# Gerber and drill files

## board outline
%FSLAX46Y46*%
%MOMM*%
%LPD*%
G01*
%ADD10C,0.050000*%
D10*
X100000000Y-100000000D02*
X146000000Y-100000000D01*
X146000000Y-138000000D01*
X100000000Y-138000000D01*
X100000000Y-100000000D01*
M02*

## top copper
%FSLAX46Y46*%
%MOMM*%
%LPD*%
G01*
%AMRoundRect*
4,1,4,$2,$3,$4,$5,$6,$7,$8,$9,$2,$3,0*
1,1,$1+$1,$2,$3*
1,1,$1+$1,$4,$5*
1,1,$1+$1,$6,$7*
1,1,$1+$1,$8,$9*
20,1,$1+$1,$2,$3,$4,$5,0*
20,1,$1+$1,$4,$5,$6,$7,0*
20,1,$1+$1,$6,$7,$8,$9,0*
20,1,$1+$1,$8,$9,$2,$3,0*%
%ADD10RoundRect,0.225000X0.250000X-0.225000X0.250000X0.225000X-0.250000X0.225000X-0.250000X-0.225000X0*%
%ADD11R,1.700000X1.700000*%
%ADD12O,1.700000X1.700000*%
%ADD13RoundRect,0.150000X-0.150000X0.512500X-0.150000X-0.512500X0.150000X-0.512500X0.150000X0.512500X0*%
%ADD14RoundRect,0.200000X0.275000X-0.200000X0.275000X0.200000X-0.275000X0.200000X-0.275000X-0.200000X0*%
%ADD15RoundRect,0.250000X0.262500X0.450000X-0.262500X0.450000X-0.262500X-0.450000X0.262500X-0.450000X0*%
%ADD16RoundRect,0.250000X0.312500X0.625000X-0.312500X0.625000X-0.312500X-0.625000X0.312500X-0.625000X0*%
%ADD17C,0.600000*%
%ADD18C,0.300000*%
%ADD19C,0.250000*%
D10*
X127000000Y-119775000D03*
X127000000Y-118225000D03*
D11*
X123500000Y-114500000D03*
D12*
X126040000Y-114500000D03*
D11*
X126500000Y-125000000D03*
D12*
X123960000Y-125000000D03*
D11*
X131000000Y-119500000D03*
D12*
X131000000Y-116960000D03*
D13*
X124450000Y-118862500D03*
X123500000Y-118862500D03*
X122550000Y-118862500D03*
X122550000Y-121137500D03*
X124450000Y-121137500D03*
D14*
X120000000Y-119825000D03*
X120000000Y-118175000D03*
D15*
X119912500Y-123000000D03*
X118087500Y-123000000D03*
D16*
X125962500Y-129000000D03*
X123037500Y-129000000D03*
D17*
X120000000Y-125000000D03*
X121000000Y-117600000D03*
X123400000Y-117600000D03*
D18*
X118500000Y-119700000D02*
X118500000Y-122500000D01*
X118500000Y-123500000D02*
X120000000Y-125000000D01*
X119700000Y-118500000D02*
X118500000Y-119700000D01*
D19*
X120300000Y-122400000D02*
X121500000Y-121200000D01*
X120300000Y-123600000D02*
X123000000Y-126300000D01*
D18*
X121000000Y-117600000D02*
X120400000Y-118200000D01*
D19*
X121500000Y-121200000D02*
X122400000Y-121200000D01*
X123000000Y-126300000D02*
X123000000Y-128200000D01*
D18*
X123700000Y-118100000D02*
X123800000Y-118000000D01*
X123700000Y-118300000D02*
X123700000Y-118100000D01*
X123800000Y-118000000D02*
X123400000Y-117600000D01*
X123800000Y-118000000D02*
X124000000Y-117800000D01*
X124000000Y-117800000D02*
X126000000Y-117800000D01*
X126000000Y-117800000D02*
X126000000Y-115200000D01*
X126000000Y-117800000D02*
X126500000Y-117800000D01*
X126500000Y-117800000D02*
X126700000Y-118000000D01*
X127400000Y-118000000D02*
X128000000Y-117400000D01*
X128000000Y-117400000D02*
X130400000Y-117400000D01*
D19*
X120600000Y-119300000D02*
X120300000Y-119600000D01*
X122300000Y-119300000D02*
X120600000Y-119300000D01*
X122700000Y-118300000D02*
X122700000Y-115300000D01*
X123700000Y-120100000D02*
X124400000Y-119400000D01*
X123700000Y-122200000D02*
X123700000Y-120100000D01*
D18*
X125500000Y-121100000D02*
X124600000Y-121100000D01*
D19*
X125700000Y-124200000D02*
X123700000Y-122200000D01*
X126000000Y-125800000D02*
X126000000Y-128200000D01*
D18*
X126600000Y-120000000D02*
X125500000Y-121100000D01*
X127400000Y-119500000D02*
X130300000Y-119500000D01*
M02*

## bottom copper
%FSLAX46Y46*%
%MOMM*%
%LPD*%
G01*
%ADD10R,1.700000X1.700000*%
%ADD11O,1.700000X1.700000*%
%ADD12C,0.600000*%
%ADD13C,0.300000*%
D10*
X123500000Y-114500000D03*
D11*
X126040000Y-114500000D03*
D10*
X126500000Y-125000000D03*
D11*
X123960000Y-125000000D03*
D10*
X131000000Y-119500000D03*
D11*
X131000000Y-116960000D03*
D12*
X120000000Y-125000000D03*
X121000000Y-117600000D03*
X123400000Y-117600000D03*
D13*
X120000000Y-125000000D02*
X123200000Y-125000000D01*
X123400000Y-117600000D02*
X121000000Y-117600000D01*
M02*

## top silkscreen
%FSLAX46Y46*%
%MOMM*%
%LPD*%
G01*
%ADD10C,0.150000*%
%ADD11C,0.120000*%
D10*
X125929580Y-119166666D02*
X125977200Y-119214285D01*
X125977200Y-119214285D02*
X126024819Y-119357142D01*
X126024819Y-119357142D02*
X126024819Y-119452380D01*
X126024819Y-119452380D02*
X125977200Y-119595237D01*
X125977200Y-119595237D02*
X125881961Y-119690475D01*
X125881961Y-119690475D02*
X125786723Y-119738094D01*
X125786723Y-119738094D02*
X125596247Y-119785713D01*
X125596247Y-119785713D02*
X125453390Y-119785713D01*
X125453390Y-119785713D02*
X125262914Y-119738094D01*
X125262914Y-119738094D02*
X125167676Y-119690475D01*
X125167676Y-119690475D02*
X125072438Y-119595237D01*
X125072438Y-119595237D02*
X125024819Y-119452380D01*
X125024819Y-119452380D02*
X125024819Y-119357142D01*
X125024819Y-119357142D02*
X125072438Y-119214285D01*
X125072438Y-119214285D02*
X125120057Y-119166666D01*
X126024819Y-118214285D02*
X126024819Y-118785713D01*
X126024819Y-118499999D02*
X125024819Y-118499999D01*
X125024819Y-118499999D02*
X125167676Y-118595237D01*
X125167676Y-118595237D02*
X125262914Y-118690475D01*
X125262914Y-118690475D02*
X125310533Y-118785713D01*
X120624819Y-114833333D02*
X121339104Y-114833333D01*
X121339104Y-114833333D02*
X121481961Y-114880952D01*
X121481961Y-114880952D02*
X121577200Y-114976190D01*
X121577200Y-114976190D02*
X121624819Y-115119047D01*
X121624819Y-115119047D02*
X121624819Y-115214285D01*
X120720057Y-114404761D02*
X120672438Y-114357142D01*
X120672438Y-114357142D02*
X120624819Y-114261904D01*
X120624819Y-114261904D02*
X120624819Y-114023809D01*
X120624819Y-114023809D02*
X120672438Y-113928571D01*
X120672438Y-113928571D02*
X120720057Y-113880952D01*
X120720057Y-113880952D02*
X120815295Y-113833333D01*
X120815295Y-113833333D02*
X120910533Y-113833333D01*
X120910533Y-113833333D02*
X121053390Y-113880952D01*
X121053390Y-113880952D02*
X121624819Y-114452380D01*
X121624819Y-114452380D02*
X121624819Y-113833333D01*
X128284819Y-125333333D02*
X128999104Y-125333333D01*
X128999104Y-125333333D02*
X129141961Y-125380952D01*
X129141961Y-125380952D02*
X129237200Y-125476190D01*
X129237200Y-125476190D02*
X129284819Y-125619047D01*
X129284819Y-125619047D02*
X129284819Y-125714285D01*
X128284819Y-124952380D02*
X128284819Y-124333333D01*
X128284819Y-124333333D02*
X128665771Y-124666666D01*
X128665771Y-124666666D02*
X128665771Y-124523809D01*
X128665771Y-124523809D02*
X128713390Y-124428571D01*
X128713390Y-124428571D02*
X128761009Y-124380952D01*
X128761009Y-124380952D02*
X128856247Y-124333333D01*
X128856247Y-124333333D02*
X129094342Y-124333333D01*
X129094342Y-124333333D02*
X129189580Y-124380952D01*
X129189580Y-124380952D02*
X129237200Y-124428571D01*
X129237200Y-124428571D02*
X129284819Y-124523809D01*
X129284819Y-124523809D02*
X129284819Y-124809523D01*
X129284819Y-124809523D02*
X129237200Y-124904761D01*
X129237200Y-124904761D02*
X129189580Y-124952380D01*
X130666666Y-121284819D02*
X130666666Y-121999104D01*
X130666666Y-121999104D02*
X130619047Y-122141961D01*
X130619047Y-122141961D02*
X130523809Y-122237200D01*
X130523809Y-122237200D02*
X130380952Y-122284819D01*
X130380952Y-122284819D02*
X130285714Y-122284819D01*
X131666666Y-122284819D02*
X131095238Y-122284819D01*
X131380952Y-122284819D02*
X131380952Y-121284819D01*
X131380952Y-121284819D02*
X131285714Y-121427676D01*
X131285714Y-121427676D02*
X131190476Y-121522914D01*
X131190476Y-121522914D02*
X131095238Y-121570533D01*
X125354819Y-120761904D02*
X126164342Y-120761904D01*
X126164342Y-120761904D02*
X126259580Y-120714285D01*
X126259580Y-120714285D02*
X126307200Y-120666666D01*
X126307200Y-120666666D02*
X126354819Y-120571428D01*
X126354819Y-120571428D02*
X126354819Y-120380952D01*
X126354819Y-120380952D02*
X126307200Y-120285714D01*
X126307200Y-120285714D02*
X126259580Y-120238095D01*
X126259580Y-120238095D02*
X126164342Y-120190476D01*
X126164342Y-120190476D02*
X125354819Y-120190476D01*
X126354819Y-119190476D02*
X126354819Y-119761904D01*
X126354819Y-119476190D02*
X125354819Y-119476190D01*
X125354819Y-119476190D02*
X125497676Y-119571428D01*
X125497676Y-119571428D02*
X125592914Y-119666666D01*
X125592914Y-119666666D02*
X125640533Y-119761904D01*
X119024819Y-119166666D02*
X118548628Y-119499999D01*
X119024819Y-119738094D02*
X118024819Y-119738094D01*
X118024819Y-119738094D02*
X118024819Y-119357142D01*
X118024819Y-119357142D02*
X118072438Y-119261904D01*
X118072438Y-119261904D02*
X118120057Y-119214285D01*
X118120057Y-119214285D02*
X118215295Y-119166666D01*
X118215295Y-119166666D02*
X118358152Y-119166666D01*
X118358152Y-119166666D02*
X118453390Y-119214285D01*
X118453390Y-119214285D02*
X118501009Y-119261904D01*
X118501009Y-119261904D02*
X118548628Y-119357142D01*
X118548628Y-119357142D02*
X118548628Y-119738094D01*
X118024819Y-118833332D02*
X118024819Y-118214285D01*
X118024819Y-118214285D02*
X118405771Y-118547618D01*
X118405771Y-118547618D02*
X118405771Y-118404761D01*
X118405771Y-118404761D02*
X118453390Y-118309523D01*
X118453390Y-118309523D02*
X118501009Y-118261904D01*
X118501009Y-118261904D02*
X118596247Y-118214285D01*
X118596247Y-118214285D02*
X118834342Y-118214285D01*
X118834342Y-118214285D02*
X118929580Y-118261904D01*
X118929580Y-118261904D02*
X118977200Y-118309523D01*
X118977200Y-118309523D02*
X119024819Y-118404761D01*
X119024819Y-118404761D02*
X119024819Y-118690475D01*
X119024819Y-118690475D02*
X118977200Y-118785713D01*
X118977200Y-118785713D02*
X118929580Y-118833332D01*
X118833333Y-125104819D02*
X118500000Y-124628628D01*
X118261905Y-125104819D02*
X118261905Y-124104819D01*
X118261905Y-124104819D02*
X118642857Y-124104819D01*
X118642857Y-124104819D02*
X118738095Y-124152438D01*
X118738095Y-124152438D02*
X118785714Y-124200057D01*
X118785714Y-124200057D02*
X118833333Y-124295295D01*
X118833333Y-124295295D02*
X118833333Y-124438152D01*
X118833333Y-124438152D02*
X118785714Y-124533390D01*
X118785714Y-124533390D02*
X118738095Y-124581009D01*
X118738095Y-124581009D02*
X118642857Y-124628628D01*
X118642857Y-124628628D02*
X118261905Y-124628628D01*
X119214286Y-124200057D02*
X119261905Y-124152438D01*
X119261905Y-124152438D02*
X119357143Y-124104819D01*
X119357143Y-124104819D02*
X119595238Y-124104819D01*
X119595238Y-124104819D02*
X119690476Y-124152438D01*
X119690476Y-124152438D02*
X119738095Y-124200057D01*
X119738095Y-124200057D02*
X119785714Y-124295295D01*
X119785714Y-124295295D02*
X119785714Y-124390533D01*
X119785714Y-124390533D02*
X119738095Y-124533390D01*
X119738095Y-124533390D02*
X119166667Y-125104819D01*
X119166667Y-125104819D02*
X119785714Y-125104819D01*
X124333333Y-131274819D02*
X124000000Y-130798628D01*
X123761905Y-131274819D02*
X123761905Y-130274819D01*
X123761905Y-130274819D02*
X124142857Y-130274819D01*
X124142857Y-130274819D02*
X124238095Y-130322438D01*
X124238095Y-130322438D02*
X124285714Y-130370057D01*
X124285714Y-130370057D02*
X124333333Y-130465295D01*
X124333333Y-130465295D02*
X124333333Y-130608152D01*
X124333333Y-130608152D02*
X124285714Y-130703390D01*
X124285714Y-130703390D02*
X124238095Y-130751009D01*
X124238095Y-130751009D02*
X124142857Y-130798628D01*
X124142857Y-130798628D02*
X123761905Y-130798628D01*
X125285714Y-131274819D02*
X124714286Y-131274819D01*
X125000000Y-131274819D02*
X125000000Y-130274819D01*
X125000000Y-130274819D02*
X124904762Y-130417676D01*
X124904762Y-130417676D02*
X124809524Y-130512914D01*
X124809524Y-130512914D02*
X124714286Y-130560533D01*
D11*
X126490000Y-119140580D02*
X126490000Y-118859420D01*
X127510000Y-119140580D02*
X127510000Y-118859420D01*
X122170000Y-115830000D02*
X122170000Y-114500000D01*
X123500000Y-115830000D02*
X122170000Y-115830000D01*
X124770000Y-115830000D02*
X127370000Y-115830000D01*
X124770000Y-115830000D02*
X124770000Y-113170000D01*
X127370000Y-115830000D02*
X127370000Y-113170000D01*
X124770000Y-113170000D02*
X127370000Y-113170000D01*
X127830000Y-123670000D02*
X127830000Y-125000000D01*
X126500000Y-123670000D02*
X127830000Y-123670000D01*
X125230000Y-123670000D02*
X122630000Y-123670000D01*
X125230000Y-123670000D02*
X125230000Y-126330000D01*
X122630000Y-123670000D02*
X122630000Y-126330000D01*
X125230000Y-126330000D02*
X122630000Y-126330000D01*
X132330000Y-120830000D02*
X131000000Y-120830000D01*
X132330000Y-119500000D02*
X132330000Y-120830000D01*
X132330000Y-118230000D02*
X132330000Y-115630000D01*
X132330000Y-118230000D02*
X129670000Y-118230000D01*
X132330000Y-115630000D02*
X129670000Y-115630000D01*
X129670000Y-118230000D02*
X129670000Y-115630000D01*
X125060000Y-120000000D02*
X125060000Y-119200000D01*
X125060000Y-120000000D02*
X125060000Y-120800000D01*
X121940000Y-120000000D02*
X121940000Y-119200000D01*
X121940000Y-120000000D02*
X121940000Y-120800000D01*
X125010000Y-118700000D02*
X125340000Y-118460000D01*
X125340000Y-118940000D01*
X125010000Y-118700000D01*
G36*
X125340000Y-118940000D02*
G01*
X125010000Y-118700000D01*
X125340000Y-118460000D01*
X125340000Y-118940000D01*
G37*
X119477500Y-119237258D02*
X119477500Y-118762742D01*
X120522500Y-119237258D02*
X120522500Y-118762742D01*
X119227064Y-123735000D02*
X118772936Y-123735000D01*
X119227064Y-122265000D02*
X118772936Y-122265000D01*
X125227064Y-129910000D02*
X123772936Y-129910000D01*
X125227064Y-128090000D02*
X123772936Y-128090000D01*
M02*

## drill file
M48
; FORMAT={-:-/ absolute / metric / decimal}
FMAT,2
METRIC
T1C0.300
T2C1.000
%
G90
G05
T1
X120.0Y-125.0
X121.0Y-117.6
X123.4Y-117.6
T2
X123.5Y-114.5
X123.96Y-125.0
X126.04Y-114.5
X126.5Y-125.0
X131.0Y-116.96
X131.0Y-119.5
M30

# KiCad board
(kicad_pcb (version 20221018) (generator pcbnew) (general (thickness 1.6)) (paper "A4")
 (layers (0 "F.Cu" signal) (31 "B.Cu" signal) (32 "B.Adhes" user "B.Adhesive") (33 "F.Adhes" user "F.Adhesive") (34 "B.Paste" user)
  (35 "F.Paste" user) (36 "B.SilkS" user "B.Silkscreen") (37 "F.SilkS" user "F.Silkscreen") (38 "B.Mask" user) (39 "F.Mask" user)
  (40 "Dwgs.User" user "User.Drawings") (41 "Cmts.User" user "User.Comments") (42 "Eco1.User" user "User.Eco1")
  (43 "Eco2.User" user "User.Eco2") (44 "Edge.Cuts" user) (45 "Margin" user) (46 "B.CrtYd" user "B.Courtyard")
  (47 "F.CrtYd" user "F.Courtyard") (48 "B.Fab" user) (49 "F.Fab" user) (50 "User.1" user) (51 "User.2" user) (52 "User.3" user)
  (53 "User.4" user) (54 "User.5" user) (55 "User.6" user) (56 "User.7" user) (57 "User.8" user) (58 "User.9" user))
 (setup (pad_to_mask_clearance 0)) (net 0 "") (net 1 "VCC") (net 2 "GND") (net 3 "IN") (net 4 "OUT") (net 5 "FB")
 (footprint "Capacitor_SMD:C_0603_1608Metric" (layer "F.Cu") (at 127 119 90)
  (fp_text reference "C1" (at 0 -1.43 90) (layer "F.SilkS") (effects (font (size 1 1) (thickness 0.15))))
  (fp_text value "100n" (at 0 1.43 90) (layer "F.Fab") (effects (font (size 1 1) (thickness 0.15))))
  (fp_line (start -0.14058 -0.51) (end 0.14058 -0.51) (stroke (width 0.12) (type solid)) (layer "F.SilkS"))
  (fp_line (start -0.14058 0.51) (end 0.14058 0.51) (stroke (width 0.12) (type solid)) (layer "F.SilkS"))
  (pad "1" smd roundrect (at -0.775 0 90) (size 0.9 0.95) (layers "F.Cu" "F.Paste" "F.Mask") (roundrect_rratio 0.25) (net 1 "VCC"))
  (pad "2" smd roundrect (at 0.775 0 90) (size 0.9 0.95) (layers "F.Cu" "F.Paste" "F.Mask") (roundrect_rratio 0.25) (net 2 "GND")))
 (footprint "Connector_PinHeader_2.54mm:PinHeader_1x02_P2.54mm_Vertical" (layer "F.Cu") (at 123.5 114.5 90)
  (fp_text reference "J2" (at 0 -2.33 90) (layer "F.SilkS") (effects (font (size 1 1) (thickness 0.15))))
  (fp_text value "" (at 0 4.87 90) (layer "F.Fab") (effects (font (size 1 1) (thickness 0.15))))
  (fp_line (start -1.33 -1.33) (end 0 -1.33) (stroke (width 0.12) (type solid)) (layer "F.SilkS"))
  (fp_line (start -1.33 0) (end -1.33 -1.33) (stroke (width 0.12) (type solid)) (layer "F.SilkS"))
  (fp_line (start -1.33 1.27) (end -1.33 3.87) (stroke (width 0.12) (type solid)) (layer "F.SilkS"))
  (fp_line (start -1.33 1.27) (end 1.33 1.27) (stroke (width 0.12) (type solid)) (layer "F.SilkS"))
  (fp_line (start -1.33 3.87) (end 1.33 3.87) (stroke (width 0.12) (type solid)) (layer "F.SilkS"))
  (fp_line (start 1.33 1.27) (end 1.33 3.87) (stroke (width 0.12) (type solid)) (layer "F.SilkS"))
  (pad "1" thru_hole rect (at 0 0 90) (size 1.7 1.7) (drill 1) (layers "*.Cu" "*.Mask") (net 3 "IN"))
  (pad "2" thru_hole oval (at 0 2.54 90) (size 1.7 1.7) (drill 1) (layers "*.Cu" "*.Mask") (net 2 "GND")))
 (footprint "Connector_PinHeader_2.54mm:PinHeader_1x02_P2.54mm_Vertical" (layer "F.Cu") (at 126.5 125 -90)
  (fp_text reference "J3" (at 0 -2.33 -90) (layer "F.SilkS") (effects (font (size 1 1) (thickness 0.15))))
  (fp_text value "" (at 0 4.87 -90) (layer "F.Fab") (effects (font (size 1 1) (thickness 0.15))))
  (fp_line (start -1.33 -1.33) (end 0 -1.33) (stroke (width 0.12) (type solid)) (layer "F.SilkS"))
  (fp_line (start -1.33 0) (end -1.33 -1.33) (stroke (width 0.12) (type solid)) (layer "F.SilkS"))
  (fp_line (start -1.33 1.27) (end -1.33 3.87) (stroke (width 0.12) (type solid)) (layer "F.SilkS"))
  (fp_line (start -1.33 1.27) (end 1.33 1.27) (stroke (width 0.12) (type solid)) (layer "F.SilkS"))
  (fp_line (start -1.33 3.87) (end 1.33 3.87) (stroke (width 0.12) (type solid)) (layer "F.SilkS"))
  (fp_line (start 1.33 1.27) (end 1.33 3.87) (stroke (width 0.12) (type solid)) (layer "F.SilkS"))
  (pad "1" thru_hole rect (at 0 0 270) (size 1.7 1.7) (drill 1) (layers "*.Cu" "*.Mask") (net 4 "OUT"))
  (pad "2" thru_hole oval (at 0 2.54 270) (size 1.7 1.7) (drill 1) (layers "*.Cu" "*.Mask") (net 2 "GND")))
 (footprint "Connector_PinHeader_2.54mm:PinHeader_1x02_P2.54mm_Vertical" (layer "F.Cu") (at 131 119.5 180)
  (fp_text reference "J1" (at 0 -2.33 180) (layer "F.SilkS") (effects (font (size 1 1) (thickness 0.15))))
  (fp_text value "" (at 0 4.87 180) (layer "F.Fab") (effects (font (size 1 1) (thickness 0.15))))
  (fp_line (start -1.33 -1.33) (end 0 -1.33) (stroke (width 0.12) (type solid)) (layer "F.SilkS"))
  (fp_line (start -1.33 0) (end -1.33 -1.33) (stroke (width 0.12) (type solid)) (layer "F.SilkS"))
  (fp_line (start -1.33 1.27) (end -1.33 3.87) (stroke (width 0.12) (type solid)) (layer "F.SilkS"))
  (fp_line (start -1.33 1.27) (end 1.33 1.27) (stroke (width 0.12) (type solid)) (layer "F.SilkS"))
  (fp_line (start -1.33 3.87) (end 1.33 3.87) (stroke (width 0.12) (type solid)) (layer "F.SilkS"))
  (fp_line (start 1.33 1.27) (end 1.33 3.87) (stroke (width 0.12) (type solid)) (layer "F.SilkS"))
  (pad "1" thru_hole rect (at 0 0 180) (size 1.7 1.7) (drill 1) (layers "*.Cu" "*.Mask") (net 1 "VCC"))
  (pad "2" thru_hole oval (at 0 2.54 180) (size 1.7 1.7) (drill 1) (layers "*.Cu" "*.Mask") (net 2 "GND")))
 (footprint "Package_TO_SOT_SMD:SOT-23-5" (layer "F.Cu") (at 123.5 120 -90)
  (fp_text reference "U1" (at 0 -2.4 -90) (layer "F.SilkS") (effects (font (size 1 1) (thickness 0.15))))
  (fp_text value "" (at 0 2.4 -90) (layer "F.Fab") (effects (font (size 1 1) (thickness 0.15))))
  (fp_line (start 0 -1.56) (end -0.8 -1.56) (stroke (width 0.12) (type solid)) (layer "F.SilkS"))
  (fp_line (start 0 -1.56) (end 0.8 -1.56) (stroke (width 0.12) (type solid)) (layer "F.SilkS"))
  (fp_line (start 0 1.56) (end -0.8 1.56) (stroke (width 0.12) (type solid)) (layer "F.SilkS"))
  (fp_line (start 0 1.56) (end 0.8 1.56) (stroke (width 0.12) (type solid)) (layer "F.SilkS"))
  (fp_poly
   (pts (xy -1.3 -1.51) (xy -1.54 -1.84) (xy -1.06 -1.84) (xy -1.3 -1.51)) (stroke (width 0.12) (type solid)) (fill solid) (layer "F.SilkS"))
  (pad "1" smd roundrect (at -1.1375 -0.95 270) (size 1.325 0.6) (layers "F.Cu" "F.Paste" "F.Mask") (roundrect_rratio 0.25) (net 4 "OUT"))
  (pad "2" smd roundrect (at -1.1375 0 270) (size 1.325 0.6) (layers "F.Cu" "F.Paste" "F.Mask") (roundrect_rratio 0.25) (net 2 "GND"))
  (pad "3" smd roundrect (at -1.1375 0.95 270) (size 1.325 0.6) (layers "F.Cu" "F.Paste" "F.Mask") (roundrect_rratio 0.25) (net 3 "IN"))
  (pad "4" smd roundrect (at 1.1375 0.95 270) (size 1.325 0.6) (layers "F.Cu" "F.Paste" "F.Mask") (roundrect_rratio 0.25) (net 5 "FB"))
  (pad "5" smd roundrect (at 1.1375 -0.95 270) (size 1.325 0.6) (layers "F.Cu" "F.Paste" "F.Mask") (roundrect_rratio 0.25) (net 1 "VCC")))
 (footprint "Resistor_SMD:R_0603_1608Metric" (layer "F.Cu") (at 120 119 90)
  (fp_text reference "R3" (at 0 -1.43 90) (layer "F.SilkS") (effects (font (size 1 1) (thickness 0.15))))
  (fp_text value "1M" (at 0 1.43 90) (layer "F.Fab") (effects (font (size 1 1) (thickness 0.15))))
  (fp_line (start -0.237258 -0.5225) (end 0.237258 -0.5225) (stroke (width 0.12) (type solid)) (layer "F.SilkS"))
  (fp_line (start -0.237258 0.5225) (end 0.237258 0.5225) (stroke (width 0.12) (type solid)) (layer "F.SilkS"))
  (pad "1" smd roundrect (at -0.825 0 90) (size 0.8 0.95) (layers "F.Cu" "F.Paste" "F.Mask") (roundrect_rratio 0.25) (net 3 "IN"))
  (pad "2" smd roundrect (at 0.825 0 90) (size 0.8 0.95) (layers "F.Cu" "F.Paste" "F.Mask") (roundrect_rratio 0.25) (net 2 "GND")))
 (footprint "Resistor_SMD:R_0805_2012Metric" (layer "F.Cu") (at 119 123 180)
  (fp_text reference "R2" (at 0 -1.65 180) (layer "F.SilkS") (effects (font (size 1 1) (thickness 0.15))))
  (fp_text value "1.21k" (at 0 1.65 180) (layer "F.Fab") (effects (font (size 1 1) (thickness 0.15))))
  (fp_line (start -0.227064 -0.735) (end 0.227064 -0.735) (stroke (width 0.12) (type solid)) (layer "F.SilkS"))
  (fp_line (start -0.227064 0.735) (end 0.227064 0.735) (stroke (width 0.12) (type solid)) (layer "F.SilkS"))
  (pad "1" smd roundrect (at -0.9125 0 180) (size 1.025 1.4) (layers "F.Cu" "F.Paste" "F.Mask") (roundrect_rratio 0.243902) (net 5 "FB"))
  (pad "2" smd roundrect (at 0.9125 0 180) (size 1.025 1.4) (layers "F.Cu" "F.Paste" "F.Mask") (roundrect_rratio 0.243902) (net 2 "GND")))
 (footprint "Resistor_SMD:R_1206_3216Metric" (layer "F.Cu") (at 124.5 129 180)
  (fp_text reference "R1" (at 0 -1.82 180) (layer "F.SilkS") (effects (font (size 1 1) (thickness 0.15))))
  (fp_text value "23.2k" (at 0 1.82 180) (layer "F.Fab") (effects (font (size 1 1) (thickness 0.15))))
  (fp_line (start -0.727064 -0.91) (end 0.727064 -0.91) (stroke (width 0.12) (type solid)) (layer "F.SilkS"))
  (fp_line (start -0.727064 0.91) (end 0.727064 0.91) (stroke (width 0.12) (type solid)) (layer "F.SilkS"))
  (pad "1" smd roundrect (at -1.4625 0 180) (size 1.125 1.75) (layers "F.Cu" "F.Paste" "F.Mask") (roundrect_rratio 0.222222) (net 4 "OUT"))
  (pad "2" smd roundrect (at 1.4625 0 180) (size 1.125 1.75) (layers "F.Cu" "F.Paste" "F.Mask") (roundrect_rratio 0.222222) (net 5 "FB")))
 (gr_rect (start 100 100) (end 146 138) (stroke (width 0.05) (type default)) (fill none) (layer "Edge.Cuts"))
 (segment (start 118.5 119.7) (end 118.5 122.5) (width 0.3) (layer "F.Cu") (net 2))
 (segment (start 118.5 123.5) (end 120 125) (width 0.3) (layer "F.Cu") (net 2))
 (segment (start 119.7 118.5) (end 118.5 119.7) (width 0.3) (layer "F.Cu") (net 2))
 (segment (start 120.3 122.4) (end 121.5 121.2) (width 0.25) (layer "F.Cu") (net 5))
 (segment (start 120.3 123.6) (end 123 126.3) (width 0.25) (layer "F.Cu") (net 5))
 (segment (start 121 117.6) (end 120.4 118.2) (width 0.3) (layer "F.Cu") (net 2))
 (segment (start 121.5 121.2) (end 122.4 121.2) (width 0.25) (layer "F.Cu") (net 5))
 (segment (start 123 126.3) (end 123 128.2) (width 0.25) (layer "F.Cu") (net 5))
 (segment (start 123.7 118.1) (end 123.8 118) (width 0.3) (layer "F.Cu") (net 2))
 (segment (start 123.7 118.3) (end 123.7 118.1) (width 0.3) (layer "F.Cu") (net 2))
 (segment (start 123.8 118) (end 123.4 117.6) (width 0.3) (layer "F.Cu") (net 2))
 (segment (start 123.8 118) (end 124 117.8) (width 0.3) (layer "F.Cu") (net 2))
 (segment (start 124 117.8) (end 126 117.8) (width 0.3) (layer "F.Cu") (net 2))
 (segment (start 126 117.8) (end 126 115.2) (width 0.3) (layer "F.Cu") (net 2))
 (segment (start 126 117.8) (end 126.5 117.8) (width 0.3) (layer "F.Cu") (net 2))
 (segment (start 126.5 117.8) (end 126.7 118) (width 0.3) (layer "F.Cu") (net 2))
 (segment (start 127.4 118) (end 128 117.4) (width 0.3) (layer "F.Cu") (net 2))
 (segment (start 128 117.4) (end 130.4 117.4) (width 0.3) (layer "F.Cu") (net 2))
 (via (at 120 125) (size 0.6) (drill 0.3) (layers "F.Cu" "B.Cu") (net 2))
 (via (at 121 117.6) (size 0.6) (drill 0.3) (layers "F.Cu" "B.Cu") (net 2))
 (via (at 123.4 117.6) (size 0.6) (drill 0.3) (layers "F.Cu" "B.Cu") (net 2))
 (segment (start 120 125) (end 123.2 125) (width 0.3) (layer "B.Cu") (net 2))
 (segment (start 120.6 119.3) (end 120.3 119.6) (width 0.25) (layer "F.Cu") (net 3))
 (segment (start 122.3 119.3) (end 120.6 119.3) (width 0.25) (layer "F.Cu") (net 3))
 (segment (start 122.7 118.3) (end 122.7 115.3) (width 0.25) (layer "F.Cu") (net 3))
 (segment (start 123.4 117.6) (end 121 117.6) (width 0.3) (layer "B.Cu") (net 2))
 (segment (start 123.7 120.1) (end 124.4 119.4) (width 0.25) (layer "F.Cu") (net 4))
 (segment (start 123.7 122.2) (end 123.7 120.1) (width 0.25) (layer "F.Cu") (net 4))
 (segment (start 125.5 121.1) (end 124.6 121.1) (width 0.3) (layer "F.Cu") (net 1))
 (segment (start 125.7 124.2) (end 123.7 122.2) (width 0.25) (layer "F.Cu") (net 4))
 (segment (start 126 125.8) (end 126 128.2) (width 0.25) (layer "F.Cu") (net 4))
 (segment (start 126.6 120) (end 125.5 121.1) (width 0.3) (layer "F.Cu") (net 1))
 (segment (start 127.4 119.5) (end 130.3 119.5) (width 0.3) (layer "F.Cu") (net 1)))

